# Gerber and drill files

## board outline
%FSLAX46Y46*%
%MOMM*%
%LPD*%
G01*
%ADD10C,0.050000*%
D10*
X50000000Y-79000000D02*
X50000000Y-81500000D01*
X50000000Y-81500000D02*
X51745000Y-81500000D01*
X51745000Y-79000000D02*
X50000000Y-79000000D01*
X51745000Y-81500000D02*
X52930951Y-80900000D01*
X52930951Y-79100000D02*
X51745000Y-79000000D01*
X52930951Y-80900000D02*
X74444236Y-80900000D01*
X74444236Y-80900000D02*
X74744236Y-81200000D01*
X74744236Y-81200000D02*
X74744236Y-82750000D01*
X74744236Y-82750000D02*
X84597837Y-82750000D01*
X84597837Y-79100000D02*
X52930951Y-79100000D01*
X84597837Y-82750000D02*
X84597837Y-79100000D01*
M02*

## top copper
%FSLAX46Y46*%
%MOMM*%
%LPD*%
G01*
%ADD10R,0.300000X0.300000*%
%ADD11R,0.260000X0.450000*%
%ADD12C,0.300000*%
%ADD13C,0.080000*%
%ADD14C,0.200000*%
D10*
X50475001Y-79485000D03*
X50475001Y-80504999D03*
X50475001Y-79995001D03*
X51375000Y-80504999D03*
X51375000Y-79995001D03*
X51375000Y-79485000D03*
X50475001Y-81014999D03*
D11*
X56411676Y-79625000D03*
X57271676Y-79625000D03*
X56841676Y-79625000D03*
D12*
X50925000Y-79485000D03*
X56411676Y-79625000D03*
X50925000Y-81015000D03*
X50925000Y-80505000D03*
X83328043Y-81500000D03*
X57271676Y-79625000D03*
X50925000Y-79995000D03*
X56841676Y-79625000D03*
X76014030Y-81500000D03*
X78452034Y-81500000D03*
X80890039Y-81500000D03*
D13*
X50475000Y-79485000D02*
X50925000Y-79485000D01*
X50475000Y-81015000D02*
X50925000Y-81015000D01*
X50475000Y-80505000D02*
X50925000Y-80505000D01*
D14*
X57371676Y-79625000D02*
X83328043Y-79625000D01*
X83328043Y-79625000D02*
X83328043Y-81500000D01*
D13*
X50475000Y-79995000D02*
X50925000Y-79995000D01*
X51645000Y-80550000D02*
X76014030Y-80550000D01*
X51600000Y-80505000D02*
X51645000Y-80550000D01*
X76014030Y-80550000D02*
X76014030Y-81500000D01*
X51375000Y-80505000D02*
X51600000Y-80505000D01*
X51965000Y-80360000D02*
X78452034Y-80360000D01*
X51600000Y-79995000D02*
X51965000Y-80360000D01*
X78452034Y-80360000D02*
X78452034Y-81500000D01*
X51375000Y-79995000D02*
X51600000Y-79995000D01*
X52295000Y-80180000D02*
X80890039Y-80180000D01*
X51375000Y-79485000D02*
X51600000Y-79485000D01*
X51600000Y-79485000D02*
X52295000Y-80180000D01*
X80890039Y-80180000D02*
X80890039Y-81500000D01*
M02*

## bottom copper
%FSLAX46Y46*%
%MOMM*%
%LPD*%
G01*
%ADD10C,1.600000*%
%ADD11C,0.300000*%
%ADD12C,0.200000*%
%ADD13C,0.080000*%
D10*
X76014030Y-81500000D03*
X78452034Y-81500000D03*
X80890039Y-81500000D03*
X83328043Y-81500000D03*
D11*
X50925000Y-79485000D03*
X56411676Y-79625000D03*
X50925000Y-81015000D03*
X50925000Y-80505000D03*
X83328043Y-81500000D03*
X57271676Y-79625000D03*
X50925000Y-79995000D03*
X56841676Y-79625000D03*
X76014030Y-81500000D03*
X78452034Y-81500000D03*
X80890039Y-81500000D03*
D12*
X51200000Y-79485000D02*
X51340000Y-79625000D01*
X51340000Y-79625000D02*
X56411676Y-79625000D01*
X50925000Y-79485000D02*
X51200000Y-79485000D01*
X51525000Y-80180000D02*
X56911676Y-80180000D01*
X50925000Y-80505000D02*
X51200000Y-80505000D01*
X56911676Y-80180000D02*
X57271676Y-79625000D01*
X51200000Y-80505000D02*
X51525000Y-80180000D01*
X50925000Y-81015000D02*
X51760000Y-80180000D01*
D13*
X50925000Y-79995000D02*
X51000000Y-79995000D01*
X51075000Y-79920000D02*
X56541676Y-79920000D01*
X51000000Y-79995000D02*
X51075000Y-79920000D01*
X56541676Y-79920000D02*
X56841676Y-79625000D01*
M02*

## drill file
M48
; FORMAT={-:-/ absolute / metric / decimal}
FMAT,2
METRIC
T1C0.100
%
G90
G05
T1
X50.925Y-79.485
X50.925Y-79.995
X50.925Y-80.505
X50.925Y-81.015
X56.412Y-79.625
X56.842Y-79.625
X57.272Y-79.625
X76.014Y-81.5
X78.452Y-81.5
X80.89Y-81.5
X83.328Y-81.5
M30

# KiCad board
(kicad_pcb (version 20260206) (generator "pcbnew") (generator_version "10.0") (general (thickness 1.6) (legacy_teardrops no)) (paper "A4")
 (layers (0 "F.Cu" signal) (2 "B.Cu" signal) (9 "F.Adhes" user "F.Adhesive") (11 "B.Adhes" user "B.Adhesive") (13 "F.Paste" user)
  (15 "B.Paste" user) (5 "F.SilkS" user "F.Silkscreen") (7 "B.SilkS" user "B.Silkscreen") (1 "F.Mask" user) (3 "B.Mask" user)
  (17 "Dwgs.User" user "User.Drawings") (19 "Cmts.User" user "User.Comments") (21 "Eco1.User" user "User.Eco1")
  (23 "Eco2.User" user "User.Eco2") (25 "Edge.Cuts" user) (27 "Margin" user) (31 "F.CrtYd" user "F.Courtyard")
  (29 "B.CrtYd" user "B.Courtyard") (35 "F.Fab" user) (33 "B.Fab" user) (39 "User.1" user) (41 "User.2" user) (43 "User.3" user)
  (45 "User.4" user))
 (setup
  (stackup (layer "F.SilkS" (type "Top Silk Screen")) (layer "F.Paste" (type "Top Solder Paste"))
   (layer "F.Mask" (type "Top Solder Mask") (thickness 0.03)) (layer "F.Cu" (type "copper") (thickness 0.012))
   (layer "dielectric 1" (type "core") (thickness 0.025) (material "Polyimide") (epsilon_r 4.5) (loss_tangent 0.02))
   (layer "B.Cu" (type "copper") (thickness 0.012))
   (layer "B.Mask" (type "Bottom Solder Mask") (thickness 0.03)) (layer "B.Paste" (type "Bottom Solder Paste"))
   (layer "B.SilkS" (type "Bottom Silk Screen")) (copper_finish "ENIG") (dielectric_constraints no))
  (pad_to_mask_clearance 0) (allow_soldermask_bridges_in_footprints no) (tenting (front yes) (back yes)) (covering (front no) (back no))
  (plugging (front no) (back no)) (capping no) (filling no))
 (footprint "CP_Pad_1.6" (layer "F.Cu") (at 76.01403 81.5)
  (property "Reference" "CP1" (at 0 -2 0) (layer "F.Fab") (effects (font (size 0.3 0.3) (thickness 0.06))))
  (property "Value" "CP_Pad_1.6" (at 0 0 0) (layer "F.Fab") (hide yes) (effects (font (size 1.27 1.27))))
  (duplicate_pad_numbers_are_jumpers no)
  (pad "1" smd circle (at 0 0) (size 1.6 1.6) (layers "B.Cu" "B.Mask") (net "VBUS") (solder_mask_margin 0.1)))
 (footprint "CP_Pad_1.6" (layer "F.Cu") (at 83.328043 81.5)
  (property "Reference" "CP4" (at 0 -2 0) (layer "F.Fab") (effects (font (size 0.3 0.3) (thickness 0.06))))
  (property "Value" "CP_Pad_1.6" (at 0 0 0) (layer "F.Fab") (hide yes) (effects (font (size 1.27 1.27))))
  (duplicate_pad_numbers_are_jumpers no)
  (pad "1" smd circle (at 0 0) (size 1.6 1.6) (layers "B.Cu" "B.Mask") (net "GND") (solder_mask_margin 0.1)))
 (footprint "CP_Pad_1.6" (layer "F.Cu") (at 80.890039 81.5)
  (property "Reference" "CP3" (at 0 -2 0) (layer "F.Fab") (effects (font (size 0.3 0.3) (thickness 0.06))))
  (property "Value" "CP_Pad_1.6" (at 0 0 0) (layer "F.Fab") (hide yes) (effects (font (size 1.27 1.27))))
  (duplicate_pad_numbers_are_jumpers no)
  (pad "1" smd circle (at 0 0) (size 1.6 1.6) (layers "B.Cu" "B.Mask") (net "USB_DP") (solder_mask_margin 0.1)))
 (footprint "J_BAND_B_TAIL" (layer "F.Cu") (at 50.9 80.25)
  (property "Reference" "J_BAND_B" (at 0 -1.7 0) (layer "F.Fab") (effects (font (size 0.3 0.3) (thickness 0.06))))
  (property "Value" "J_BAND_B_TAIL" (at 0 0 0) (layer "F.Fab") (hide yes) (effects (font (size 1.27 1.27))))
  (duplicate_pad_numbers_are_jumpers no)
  (pad "1" smd rect (at -0.424999 -0.765) (size 0.3 0.3) (layers "F.Cu" "F.Mask") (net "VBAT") (solder_mask_margin 0.05)
   (thermal_bridge_angle 45))
  (pad "2" smd rect (at -0.424999 0.254999) (size 0.3 0.3) (layers "F.Cu" "F.Mask") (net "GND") (solder_mask_margin 0.05)
   (thermal_bridge_angle 45))
  (pad "3" smd rect (at -0.424999 -0.254999) (size 0.3 0.3) (layers "F.Cu" "F.Mask") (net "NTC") (solder_mask_margin 0.05)
   (thermal_bridge_angle 45))
  (pad "4" smd rect (at 0.475 0.254999) (size 0.3 0.3) (layers "F.Cu" "F.Mask") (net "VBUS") (solder_mask_margin 0.05)
   (thermal_bridge_angle 45))
  (pad "5" smd rect (at 0.475 -0.254999) (size 0.3 0.3) (layers "F.Cu" "F.Mask") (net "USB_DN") (solder_mask_margin 0.05)
   (thermal_bridge_angle 45))
  (pad "6" smd rect (at 0.475 -0.765) (size 0.3 0.3) (layers "F.Cu" "F.Mask") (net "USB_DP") (solder_mask_margin 0.05)
   (thermal_bridge_angle 45))
  (pad "7" smd rect (at -0.424999 0.764999) (size 0.3 0.3) (layers "F.Cu" "F.Mask") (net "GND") (solder_mask_margin 0.05)
   (thermal_bridge_angle 45)))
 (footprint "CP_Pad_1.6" (layer "F.Cu") (at 78.452034 81.5)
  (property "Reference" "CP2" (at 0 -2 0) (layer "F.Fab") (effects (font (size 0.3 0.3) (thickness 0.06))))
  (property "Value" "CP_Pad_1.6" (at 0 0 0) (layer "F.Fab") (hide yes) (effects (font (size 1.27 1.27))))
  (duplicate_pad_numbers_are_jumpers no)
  (pad "1" smd circle (at 0 0) (size 1.6 1.6) (layers "B.Cu" "B.Mask") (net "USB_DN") (solder_mask_margin 0.1)))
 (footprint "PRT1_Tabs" (layer "F.Cu") (at 56.841676 79.625)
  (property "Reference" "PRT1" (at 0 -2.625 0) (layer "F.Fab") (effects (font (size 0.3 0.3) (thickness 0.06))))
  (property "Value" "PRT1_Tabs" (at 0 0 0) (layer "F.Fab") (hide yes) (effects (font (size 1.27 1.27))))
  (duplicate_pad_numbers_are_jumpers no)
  (pad "1" smd rect (at -0.43 0) (size 0.26 0.45) (layers "F.Cu" "F.Mask") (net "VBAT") (solder_mask_margin 0.05) (thermal_bridge_angle 45))
  (pad "2" smd rect (at 0.43 0) (size 0.26 0.45) (layers "F.Cu" "F.Mask") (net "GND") (solder_mask_margin 0.05) (thermal_bridge_angle 45))
  (pad "3" smd rect (at 0 0) (size 0.26 0.45) (layers "F.Cu" "F.Mask") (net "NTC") (solder_mask_margin 0.05) (thermal_bridge_angle 45)))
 (gr_line (start 50 79) (end 50 81.5) (stroke (width 0.05) (type default)) (layer "Edge.Cuts"))
 (gr_line (start 50 81.5) (end 51.745 81.5) (stroke (width 0.05) (type default)) (layer "Edge.Cuts"))
 (gr_line (start 51.745 79) (end 50 79) (stroke (width 0.05) (type default)) (layer "Edge.Cuts"))
 (gr_line (start 51.745 81.5) (end 52.930951 80.9) (stroke (width 0.05) (type default)) (layer "Edge.Cuts"))
 (gr_line (start 52.930951 79.1) (end 51.745 79) (stroke (width 0.05) (type default)) (layer "Edge.Cuts"))
 (gr_line (start 52.930951 80.9) (end 74.444236 80.9) (stroke (width 0.05) (type default)) (layer "Edge.Cuts"))
 (gr_line (start 74.444236 80.9) (end 74.744236 81.2) (stroke (width 0.05) (type default)) (layer "Edge.Cuts"))
 (gr_line (start 74.744236 81.2) (end 74.744236 82.75) (stroke (width 0.05) (type default)) (layer "Edge.Cuts"))
 (gr_line (start 74.744236 82.75) (end 84.597837 82.75) (stroke (width 0.05) (type default)) (layer "Edge.Cuts"))
 (gr_line (start 84.597837 79.1) (end 52.930951 79.1) (stroke (width 0.05) (type default)) (layer "Edge.Cuts"))
 (gr_line (start 84.597837 82.75) (end 84.597837 79.1) (stroke (width 0.05) (type default)) (layer "Edge.Cuts"))
 (segment (start 51.375 80.505) (end 51.6 80.505) (width 0.08) (layer "F.Cu") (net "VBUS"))
 (segment (start 51.645 80.55) (end 76.01403 80.55) (width 0.08) (layer "F.Cu") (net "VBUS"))
 (segment (start 76.01403 80.55) (end 76.01403 81.5) (width 0.08) (layer "F.Cu") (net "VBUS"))
 (segment (start 51.6 80.505) (end 51.645 80.55) (width 0.08) (layer "F.Cu") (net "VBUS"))
 (via (at 76.01403 81.5) (size 0.3) (drill 0.1) (layers "F.Cu" "B.Cu") (tenting (front yes) (back yes)) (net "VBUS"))
 (segment (start 57.371676 79.625) (end 83.328043 79.625) (width 0.2) (layer "F.Cu") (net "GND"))
 (segment (start 50.475 81.015) (end 50.925 81.015) (width 0.08) (layer "F.Cu") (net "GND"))
 (segment (start 50.475 80.505) (end 50.925 80.505) (width 0.08) (layer "F.Cu") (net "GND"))
 (segment (start 83.328043 79.625) (end 83.328043 81.5) (width 0.2) (layer "F.Cu") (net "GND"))
 (via (at 57.271676 79.625) (size 0.3) (drill 0.1) (layers "F.Cu" "B.Cu") (tenting (front yes) (back yes)) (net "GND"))
 (via (at 50.925 80.505) (size 0.3) (drill 0.1) (layers "F.Cu" "B.Cu") (tenting (front yes) (back yes)) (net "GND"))
 (via (at 50.925 81.015) (size 0.3) (drill 0.1) (layers "F.Cu" "B.Cu") (tenting (front yes) (back yes)) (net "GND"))
 (via (at 83.328043 81.5) (size 0.3) (drill 0.1) (layers "F.Cu" "B.Cu") (tenting (front yes) (back yes)) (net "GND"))
 (segment (start 50.925 80.505) (end 51.2 80.505) (width 0.2) (layer "B.Cu") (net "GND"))
 (segment (start 51.525 80.18) (end 56.911676 80.18) (width 0.2) (layer "B.Cu") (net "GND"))
 (segment (start 51.2 80.505) (end 51.525 80.18) (width 0.2) (layer "B.Cu") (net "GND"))
 (segment (start 56.911676 80.18) (end 57.271676 79.625) (width 0.2) (layer "B.Cu") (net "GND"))
 (segment (start 50.925 81.015) (end 51.76 80.18) (width 0.2) (layer "B.Cu") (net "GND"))
 (segment (start 52.295 80.18) (end 80.890039 80.18) (width 0.08) (layer "F.Cu") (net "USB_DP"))
 (segment (start 51.6 79.485) (end 52.295 80.18) (width 0.08) (layer "F.Cu") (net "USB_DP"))
 (segment (start 80.890039 80.18) (end 80.890039 81.5) (width 0.08) (layer "F.Cu") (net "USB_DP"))
 (segment (start 51.375 79.485) (end 51.6 79.485) (width 0.08) (layer "F.Cu") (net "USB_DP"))
 (via (at 80.890039 81.5) (size 0.3) (drill 0.1) (layers "F.Cu" "B.Cu") (tenting (front yes) (back yes)) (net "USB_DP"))
 (segment (start 50.475 79.485) (end 50.925 79.485) (width 0.08) (layer "F.Cu") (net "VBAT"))
 (via (at 50.925 79.485) (size 0.3) (drill 0.1) (layers "F.Cu" "B.Cu") (tenting (front yes) (back yes)) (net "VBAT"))
 (via (at 56.411676 79.625) (size 0.3) (drill 0.1) (layers "F.Cu" "B.Cu") (tenting (front yes) (back yes)) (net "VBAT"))
 (segment (start 50.925 79.485) (end 51.2 79.485) (width 0.2) (layer "B.Cu") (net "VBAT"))
 (segment (start 51.34 79.625) (end 56.411676 79.625) (width 0.2) (layer "B.Cu") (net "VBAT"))
 (segment (start 51.2 79.485) (end 51.34 79.625) (width 0.2) (layer "B.Cu") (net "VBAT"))
 (segment (start 50.475 79.995) (end 50.925 79.995) (width 0.08) (layer "F.Cu") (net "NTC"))
 (via (at 50.925 79.995) (size 0.3) (drill 0.1) (layers "F.Cu" "B.Cu") (tenting (front yes) (back yes)) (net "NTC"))
 (via (at 56.841676 79.625) (size 0.3) (drill 0.1) (layers "F.Cu" "B.Cu") (tenting (front yes) (back yes)) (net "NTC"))
 (segment (start 51 79.995) (end 51.075 79.92) (width 0.08) (layer "B.Cu") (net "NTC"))
 (segment (start 56.541676 79.92) (end 56.841676 79.625) (width 0.08) (layer "B.Cu") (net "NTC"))
 (segment (start 51.075 79.92) (end 56.541676 79.92) (width 0.08) (layer "B.Cu") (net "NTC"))
 (segment (start 50.925 79.995) (end 51 79.995) (width 0.08) (layer "B.Cu") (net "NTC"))
 (segment (start 51.375 79.995) (end 51.6 79.995) (width 0.08) (layer "F.Cu") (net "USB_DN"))
 (segment (start 51.6 79.995) (end 51.965 80.36) (width 0.08) (layer "F.Cu") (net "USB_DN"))
 (segment (start 51.965 80.36) (end 78.452034 80.36) (width 0.08) (layer "F.Cu") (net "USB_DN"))
 (segment (start 78.452034 80.36) (end 78.452034 81.5) (width 0.08) (layer "F.Cu") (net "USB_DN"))
 (via (at 78.452034 81.5) (size 0.3) (drill 0.1) (layers "F.Cu" "B.Cu") (tenting (front yes) (back yes)) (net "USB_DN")))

